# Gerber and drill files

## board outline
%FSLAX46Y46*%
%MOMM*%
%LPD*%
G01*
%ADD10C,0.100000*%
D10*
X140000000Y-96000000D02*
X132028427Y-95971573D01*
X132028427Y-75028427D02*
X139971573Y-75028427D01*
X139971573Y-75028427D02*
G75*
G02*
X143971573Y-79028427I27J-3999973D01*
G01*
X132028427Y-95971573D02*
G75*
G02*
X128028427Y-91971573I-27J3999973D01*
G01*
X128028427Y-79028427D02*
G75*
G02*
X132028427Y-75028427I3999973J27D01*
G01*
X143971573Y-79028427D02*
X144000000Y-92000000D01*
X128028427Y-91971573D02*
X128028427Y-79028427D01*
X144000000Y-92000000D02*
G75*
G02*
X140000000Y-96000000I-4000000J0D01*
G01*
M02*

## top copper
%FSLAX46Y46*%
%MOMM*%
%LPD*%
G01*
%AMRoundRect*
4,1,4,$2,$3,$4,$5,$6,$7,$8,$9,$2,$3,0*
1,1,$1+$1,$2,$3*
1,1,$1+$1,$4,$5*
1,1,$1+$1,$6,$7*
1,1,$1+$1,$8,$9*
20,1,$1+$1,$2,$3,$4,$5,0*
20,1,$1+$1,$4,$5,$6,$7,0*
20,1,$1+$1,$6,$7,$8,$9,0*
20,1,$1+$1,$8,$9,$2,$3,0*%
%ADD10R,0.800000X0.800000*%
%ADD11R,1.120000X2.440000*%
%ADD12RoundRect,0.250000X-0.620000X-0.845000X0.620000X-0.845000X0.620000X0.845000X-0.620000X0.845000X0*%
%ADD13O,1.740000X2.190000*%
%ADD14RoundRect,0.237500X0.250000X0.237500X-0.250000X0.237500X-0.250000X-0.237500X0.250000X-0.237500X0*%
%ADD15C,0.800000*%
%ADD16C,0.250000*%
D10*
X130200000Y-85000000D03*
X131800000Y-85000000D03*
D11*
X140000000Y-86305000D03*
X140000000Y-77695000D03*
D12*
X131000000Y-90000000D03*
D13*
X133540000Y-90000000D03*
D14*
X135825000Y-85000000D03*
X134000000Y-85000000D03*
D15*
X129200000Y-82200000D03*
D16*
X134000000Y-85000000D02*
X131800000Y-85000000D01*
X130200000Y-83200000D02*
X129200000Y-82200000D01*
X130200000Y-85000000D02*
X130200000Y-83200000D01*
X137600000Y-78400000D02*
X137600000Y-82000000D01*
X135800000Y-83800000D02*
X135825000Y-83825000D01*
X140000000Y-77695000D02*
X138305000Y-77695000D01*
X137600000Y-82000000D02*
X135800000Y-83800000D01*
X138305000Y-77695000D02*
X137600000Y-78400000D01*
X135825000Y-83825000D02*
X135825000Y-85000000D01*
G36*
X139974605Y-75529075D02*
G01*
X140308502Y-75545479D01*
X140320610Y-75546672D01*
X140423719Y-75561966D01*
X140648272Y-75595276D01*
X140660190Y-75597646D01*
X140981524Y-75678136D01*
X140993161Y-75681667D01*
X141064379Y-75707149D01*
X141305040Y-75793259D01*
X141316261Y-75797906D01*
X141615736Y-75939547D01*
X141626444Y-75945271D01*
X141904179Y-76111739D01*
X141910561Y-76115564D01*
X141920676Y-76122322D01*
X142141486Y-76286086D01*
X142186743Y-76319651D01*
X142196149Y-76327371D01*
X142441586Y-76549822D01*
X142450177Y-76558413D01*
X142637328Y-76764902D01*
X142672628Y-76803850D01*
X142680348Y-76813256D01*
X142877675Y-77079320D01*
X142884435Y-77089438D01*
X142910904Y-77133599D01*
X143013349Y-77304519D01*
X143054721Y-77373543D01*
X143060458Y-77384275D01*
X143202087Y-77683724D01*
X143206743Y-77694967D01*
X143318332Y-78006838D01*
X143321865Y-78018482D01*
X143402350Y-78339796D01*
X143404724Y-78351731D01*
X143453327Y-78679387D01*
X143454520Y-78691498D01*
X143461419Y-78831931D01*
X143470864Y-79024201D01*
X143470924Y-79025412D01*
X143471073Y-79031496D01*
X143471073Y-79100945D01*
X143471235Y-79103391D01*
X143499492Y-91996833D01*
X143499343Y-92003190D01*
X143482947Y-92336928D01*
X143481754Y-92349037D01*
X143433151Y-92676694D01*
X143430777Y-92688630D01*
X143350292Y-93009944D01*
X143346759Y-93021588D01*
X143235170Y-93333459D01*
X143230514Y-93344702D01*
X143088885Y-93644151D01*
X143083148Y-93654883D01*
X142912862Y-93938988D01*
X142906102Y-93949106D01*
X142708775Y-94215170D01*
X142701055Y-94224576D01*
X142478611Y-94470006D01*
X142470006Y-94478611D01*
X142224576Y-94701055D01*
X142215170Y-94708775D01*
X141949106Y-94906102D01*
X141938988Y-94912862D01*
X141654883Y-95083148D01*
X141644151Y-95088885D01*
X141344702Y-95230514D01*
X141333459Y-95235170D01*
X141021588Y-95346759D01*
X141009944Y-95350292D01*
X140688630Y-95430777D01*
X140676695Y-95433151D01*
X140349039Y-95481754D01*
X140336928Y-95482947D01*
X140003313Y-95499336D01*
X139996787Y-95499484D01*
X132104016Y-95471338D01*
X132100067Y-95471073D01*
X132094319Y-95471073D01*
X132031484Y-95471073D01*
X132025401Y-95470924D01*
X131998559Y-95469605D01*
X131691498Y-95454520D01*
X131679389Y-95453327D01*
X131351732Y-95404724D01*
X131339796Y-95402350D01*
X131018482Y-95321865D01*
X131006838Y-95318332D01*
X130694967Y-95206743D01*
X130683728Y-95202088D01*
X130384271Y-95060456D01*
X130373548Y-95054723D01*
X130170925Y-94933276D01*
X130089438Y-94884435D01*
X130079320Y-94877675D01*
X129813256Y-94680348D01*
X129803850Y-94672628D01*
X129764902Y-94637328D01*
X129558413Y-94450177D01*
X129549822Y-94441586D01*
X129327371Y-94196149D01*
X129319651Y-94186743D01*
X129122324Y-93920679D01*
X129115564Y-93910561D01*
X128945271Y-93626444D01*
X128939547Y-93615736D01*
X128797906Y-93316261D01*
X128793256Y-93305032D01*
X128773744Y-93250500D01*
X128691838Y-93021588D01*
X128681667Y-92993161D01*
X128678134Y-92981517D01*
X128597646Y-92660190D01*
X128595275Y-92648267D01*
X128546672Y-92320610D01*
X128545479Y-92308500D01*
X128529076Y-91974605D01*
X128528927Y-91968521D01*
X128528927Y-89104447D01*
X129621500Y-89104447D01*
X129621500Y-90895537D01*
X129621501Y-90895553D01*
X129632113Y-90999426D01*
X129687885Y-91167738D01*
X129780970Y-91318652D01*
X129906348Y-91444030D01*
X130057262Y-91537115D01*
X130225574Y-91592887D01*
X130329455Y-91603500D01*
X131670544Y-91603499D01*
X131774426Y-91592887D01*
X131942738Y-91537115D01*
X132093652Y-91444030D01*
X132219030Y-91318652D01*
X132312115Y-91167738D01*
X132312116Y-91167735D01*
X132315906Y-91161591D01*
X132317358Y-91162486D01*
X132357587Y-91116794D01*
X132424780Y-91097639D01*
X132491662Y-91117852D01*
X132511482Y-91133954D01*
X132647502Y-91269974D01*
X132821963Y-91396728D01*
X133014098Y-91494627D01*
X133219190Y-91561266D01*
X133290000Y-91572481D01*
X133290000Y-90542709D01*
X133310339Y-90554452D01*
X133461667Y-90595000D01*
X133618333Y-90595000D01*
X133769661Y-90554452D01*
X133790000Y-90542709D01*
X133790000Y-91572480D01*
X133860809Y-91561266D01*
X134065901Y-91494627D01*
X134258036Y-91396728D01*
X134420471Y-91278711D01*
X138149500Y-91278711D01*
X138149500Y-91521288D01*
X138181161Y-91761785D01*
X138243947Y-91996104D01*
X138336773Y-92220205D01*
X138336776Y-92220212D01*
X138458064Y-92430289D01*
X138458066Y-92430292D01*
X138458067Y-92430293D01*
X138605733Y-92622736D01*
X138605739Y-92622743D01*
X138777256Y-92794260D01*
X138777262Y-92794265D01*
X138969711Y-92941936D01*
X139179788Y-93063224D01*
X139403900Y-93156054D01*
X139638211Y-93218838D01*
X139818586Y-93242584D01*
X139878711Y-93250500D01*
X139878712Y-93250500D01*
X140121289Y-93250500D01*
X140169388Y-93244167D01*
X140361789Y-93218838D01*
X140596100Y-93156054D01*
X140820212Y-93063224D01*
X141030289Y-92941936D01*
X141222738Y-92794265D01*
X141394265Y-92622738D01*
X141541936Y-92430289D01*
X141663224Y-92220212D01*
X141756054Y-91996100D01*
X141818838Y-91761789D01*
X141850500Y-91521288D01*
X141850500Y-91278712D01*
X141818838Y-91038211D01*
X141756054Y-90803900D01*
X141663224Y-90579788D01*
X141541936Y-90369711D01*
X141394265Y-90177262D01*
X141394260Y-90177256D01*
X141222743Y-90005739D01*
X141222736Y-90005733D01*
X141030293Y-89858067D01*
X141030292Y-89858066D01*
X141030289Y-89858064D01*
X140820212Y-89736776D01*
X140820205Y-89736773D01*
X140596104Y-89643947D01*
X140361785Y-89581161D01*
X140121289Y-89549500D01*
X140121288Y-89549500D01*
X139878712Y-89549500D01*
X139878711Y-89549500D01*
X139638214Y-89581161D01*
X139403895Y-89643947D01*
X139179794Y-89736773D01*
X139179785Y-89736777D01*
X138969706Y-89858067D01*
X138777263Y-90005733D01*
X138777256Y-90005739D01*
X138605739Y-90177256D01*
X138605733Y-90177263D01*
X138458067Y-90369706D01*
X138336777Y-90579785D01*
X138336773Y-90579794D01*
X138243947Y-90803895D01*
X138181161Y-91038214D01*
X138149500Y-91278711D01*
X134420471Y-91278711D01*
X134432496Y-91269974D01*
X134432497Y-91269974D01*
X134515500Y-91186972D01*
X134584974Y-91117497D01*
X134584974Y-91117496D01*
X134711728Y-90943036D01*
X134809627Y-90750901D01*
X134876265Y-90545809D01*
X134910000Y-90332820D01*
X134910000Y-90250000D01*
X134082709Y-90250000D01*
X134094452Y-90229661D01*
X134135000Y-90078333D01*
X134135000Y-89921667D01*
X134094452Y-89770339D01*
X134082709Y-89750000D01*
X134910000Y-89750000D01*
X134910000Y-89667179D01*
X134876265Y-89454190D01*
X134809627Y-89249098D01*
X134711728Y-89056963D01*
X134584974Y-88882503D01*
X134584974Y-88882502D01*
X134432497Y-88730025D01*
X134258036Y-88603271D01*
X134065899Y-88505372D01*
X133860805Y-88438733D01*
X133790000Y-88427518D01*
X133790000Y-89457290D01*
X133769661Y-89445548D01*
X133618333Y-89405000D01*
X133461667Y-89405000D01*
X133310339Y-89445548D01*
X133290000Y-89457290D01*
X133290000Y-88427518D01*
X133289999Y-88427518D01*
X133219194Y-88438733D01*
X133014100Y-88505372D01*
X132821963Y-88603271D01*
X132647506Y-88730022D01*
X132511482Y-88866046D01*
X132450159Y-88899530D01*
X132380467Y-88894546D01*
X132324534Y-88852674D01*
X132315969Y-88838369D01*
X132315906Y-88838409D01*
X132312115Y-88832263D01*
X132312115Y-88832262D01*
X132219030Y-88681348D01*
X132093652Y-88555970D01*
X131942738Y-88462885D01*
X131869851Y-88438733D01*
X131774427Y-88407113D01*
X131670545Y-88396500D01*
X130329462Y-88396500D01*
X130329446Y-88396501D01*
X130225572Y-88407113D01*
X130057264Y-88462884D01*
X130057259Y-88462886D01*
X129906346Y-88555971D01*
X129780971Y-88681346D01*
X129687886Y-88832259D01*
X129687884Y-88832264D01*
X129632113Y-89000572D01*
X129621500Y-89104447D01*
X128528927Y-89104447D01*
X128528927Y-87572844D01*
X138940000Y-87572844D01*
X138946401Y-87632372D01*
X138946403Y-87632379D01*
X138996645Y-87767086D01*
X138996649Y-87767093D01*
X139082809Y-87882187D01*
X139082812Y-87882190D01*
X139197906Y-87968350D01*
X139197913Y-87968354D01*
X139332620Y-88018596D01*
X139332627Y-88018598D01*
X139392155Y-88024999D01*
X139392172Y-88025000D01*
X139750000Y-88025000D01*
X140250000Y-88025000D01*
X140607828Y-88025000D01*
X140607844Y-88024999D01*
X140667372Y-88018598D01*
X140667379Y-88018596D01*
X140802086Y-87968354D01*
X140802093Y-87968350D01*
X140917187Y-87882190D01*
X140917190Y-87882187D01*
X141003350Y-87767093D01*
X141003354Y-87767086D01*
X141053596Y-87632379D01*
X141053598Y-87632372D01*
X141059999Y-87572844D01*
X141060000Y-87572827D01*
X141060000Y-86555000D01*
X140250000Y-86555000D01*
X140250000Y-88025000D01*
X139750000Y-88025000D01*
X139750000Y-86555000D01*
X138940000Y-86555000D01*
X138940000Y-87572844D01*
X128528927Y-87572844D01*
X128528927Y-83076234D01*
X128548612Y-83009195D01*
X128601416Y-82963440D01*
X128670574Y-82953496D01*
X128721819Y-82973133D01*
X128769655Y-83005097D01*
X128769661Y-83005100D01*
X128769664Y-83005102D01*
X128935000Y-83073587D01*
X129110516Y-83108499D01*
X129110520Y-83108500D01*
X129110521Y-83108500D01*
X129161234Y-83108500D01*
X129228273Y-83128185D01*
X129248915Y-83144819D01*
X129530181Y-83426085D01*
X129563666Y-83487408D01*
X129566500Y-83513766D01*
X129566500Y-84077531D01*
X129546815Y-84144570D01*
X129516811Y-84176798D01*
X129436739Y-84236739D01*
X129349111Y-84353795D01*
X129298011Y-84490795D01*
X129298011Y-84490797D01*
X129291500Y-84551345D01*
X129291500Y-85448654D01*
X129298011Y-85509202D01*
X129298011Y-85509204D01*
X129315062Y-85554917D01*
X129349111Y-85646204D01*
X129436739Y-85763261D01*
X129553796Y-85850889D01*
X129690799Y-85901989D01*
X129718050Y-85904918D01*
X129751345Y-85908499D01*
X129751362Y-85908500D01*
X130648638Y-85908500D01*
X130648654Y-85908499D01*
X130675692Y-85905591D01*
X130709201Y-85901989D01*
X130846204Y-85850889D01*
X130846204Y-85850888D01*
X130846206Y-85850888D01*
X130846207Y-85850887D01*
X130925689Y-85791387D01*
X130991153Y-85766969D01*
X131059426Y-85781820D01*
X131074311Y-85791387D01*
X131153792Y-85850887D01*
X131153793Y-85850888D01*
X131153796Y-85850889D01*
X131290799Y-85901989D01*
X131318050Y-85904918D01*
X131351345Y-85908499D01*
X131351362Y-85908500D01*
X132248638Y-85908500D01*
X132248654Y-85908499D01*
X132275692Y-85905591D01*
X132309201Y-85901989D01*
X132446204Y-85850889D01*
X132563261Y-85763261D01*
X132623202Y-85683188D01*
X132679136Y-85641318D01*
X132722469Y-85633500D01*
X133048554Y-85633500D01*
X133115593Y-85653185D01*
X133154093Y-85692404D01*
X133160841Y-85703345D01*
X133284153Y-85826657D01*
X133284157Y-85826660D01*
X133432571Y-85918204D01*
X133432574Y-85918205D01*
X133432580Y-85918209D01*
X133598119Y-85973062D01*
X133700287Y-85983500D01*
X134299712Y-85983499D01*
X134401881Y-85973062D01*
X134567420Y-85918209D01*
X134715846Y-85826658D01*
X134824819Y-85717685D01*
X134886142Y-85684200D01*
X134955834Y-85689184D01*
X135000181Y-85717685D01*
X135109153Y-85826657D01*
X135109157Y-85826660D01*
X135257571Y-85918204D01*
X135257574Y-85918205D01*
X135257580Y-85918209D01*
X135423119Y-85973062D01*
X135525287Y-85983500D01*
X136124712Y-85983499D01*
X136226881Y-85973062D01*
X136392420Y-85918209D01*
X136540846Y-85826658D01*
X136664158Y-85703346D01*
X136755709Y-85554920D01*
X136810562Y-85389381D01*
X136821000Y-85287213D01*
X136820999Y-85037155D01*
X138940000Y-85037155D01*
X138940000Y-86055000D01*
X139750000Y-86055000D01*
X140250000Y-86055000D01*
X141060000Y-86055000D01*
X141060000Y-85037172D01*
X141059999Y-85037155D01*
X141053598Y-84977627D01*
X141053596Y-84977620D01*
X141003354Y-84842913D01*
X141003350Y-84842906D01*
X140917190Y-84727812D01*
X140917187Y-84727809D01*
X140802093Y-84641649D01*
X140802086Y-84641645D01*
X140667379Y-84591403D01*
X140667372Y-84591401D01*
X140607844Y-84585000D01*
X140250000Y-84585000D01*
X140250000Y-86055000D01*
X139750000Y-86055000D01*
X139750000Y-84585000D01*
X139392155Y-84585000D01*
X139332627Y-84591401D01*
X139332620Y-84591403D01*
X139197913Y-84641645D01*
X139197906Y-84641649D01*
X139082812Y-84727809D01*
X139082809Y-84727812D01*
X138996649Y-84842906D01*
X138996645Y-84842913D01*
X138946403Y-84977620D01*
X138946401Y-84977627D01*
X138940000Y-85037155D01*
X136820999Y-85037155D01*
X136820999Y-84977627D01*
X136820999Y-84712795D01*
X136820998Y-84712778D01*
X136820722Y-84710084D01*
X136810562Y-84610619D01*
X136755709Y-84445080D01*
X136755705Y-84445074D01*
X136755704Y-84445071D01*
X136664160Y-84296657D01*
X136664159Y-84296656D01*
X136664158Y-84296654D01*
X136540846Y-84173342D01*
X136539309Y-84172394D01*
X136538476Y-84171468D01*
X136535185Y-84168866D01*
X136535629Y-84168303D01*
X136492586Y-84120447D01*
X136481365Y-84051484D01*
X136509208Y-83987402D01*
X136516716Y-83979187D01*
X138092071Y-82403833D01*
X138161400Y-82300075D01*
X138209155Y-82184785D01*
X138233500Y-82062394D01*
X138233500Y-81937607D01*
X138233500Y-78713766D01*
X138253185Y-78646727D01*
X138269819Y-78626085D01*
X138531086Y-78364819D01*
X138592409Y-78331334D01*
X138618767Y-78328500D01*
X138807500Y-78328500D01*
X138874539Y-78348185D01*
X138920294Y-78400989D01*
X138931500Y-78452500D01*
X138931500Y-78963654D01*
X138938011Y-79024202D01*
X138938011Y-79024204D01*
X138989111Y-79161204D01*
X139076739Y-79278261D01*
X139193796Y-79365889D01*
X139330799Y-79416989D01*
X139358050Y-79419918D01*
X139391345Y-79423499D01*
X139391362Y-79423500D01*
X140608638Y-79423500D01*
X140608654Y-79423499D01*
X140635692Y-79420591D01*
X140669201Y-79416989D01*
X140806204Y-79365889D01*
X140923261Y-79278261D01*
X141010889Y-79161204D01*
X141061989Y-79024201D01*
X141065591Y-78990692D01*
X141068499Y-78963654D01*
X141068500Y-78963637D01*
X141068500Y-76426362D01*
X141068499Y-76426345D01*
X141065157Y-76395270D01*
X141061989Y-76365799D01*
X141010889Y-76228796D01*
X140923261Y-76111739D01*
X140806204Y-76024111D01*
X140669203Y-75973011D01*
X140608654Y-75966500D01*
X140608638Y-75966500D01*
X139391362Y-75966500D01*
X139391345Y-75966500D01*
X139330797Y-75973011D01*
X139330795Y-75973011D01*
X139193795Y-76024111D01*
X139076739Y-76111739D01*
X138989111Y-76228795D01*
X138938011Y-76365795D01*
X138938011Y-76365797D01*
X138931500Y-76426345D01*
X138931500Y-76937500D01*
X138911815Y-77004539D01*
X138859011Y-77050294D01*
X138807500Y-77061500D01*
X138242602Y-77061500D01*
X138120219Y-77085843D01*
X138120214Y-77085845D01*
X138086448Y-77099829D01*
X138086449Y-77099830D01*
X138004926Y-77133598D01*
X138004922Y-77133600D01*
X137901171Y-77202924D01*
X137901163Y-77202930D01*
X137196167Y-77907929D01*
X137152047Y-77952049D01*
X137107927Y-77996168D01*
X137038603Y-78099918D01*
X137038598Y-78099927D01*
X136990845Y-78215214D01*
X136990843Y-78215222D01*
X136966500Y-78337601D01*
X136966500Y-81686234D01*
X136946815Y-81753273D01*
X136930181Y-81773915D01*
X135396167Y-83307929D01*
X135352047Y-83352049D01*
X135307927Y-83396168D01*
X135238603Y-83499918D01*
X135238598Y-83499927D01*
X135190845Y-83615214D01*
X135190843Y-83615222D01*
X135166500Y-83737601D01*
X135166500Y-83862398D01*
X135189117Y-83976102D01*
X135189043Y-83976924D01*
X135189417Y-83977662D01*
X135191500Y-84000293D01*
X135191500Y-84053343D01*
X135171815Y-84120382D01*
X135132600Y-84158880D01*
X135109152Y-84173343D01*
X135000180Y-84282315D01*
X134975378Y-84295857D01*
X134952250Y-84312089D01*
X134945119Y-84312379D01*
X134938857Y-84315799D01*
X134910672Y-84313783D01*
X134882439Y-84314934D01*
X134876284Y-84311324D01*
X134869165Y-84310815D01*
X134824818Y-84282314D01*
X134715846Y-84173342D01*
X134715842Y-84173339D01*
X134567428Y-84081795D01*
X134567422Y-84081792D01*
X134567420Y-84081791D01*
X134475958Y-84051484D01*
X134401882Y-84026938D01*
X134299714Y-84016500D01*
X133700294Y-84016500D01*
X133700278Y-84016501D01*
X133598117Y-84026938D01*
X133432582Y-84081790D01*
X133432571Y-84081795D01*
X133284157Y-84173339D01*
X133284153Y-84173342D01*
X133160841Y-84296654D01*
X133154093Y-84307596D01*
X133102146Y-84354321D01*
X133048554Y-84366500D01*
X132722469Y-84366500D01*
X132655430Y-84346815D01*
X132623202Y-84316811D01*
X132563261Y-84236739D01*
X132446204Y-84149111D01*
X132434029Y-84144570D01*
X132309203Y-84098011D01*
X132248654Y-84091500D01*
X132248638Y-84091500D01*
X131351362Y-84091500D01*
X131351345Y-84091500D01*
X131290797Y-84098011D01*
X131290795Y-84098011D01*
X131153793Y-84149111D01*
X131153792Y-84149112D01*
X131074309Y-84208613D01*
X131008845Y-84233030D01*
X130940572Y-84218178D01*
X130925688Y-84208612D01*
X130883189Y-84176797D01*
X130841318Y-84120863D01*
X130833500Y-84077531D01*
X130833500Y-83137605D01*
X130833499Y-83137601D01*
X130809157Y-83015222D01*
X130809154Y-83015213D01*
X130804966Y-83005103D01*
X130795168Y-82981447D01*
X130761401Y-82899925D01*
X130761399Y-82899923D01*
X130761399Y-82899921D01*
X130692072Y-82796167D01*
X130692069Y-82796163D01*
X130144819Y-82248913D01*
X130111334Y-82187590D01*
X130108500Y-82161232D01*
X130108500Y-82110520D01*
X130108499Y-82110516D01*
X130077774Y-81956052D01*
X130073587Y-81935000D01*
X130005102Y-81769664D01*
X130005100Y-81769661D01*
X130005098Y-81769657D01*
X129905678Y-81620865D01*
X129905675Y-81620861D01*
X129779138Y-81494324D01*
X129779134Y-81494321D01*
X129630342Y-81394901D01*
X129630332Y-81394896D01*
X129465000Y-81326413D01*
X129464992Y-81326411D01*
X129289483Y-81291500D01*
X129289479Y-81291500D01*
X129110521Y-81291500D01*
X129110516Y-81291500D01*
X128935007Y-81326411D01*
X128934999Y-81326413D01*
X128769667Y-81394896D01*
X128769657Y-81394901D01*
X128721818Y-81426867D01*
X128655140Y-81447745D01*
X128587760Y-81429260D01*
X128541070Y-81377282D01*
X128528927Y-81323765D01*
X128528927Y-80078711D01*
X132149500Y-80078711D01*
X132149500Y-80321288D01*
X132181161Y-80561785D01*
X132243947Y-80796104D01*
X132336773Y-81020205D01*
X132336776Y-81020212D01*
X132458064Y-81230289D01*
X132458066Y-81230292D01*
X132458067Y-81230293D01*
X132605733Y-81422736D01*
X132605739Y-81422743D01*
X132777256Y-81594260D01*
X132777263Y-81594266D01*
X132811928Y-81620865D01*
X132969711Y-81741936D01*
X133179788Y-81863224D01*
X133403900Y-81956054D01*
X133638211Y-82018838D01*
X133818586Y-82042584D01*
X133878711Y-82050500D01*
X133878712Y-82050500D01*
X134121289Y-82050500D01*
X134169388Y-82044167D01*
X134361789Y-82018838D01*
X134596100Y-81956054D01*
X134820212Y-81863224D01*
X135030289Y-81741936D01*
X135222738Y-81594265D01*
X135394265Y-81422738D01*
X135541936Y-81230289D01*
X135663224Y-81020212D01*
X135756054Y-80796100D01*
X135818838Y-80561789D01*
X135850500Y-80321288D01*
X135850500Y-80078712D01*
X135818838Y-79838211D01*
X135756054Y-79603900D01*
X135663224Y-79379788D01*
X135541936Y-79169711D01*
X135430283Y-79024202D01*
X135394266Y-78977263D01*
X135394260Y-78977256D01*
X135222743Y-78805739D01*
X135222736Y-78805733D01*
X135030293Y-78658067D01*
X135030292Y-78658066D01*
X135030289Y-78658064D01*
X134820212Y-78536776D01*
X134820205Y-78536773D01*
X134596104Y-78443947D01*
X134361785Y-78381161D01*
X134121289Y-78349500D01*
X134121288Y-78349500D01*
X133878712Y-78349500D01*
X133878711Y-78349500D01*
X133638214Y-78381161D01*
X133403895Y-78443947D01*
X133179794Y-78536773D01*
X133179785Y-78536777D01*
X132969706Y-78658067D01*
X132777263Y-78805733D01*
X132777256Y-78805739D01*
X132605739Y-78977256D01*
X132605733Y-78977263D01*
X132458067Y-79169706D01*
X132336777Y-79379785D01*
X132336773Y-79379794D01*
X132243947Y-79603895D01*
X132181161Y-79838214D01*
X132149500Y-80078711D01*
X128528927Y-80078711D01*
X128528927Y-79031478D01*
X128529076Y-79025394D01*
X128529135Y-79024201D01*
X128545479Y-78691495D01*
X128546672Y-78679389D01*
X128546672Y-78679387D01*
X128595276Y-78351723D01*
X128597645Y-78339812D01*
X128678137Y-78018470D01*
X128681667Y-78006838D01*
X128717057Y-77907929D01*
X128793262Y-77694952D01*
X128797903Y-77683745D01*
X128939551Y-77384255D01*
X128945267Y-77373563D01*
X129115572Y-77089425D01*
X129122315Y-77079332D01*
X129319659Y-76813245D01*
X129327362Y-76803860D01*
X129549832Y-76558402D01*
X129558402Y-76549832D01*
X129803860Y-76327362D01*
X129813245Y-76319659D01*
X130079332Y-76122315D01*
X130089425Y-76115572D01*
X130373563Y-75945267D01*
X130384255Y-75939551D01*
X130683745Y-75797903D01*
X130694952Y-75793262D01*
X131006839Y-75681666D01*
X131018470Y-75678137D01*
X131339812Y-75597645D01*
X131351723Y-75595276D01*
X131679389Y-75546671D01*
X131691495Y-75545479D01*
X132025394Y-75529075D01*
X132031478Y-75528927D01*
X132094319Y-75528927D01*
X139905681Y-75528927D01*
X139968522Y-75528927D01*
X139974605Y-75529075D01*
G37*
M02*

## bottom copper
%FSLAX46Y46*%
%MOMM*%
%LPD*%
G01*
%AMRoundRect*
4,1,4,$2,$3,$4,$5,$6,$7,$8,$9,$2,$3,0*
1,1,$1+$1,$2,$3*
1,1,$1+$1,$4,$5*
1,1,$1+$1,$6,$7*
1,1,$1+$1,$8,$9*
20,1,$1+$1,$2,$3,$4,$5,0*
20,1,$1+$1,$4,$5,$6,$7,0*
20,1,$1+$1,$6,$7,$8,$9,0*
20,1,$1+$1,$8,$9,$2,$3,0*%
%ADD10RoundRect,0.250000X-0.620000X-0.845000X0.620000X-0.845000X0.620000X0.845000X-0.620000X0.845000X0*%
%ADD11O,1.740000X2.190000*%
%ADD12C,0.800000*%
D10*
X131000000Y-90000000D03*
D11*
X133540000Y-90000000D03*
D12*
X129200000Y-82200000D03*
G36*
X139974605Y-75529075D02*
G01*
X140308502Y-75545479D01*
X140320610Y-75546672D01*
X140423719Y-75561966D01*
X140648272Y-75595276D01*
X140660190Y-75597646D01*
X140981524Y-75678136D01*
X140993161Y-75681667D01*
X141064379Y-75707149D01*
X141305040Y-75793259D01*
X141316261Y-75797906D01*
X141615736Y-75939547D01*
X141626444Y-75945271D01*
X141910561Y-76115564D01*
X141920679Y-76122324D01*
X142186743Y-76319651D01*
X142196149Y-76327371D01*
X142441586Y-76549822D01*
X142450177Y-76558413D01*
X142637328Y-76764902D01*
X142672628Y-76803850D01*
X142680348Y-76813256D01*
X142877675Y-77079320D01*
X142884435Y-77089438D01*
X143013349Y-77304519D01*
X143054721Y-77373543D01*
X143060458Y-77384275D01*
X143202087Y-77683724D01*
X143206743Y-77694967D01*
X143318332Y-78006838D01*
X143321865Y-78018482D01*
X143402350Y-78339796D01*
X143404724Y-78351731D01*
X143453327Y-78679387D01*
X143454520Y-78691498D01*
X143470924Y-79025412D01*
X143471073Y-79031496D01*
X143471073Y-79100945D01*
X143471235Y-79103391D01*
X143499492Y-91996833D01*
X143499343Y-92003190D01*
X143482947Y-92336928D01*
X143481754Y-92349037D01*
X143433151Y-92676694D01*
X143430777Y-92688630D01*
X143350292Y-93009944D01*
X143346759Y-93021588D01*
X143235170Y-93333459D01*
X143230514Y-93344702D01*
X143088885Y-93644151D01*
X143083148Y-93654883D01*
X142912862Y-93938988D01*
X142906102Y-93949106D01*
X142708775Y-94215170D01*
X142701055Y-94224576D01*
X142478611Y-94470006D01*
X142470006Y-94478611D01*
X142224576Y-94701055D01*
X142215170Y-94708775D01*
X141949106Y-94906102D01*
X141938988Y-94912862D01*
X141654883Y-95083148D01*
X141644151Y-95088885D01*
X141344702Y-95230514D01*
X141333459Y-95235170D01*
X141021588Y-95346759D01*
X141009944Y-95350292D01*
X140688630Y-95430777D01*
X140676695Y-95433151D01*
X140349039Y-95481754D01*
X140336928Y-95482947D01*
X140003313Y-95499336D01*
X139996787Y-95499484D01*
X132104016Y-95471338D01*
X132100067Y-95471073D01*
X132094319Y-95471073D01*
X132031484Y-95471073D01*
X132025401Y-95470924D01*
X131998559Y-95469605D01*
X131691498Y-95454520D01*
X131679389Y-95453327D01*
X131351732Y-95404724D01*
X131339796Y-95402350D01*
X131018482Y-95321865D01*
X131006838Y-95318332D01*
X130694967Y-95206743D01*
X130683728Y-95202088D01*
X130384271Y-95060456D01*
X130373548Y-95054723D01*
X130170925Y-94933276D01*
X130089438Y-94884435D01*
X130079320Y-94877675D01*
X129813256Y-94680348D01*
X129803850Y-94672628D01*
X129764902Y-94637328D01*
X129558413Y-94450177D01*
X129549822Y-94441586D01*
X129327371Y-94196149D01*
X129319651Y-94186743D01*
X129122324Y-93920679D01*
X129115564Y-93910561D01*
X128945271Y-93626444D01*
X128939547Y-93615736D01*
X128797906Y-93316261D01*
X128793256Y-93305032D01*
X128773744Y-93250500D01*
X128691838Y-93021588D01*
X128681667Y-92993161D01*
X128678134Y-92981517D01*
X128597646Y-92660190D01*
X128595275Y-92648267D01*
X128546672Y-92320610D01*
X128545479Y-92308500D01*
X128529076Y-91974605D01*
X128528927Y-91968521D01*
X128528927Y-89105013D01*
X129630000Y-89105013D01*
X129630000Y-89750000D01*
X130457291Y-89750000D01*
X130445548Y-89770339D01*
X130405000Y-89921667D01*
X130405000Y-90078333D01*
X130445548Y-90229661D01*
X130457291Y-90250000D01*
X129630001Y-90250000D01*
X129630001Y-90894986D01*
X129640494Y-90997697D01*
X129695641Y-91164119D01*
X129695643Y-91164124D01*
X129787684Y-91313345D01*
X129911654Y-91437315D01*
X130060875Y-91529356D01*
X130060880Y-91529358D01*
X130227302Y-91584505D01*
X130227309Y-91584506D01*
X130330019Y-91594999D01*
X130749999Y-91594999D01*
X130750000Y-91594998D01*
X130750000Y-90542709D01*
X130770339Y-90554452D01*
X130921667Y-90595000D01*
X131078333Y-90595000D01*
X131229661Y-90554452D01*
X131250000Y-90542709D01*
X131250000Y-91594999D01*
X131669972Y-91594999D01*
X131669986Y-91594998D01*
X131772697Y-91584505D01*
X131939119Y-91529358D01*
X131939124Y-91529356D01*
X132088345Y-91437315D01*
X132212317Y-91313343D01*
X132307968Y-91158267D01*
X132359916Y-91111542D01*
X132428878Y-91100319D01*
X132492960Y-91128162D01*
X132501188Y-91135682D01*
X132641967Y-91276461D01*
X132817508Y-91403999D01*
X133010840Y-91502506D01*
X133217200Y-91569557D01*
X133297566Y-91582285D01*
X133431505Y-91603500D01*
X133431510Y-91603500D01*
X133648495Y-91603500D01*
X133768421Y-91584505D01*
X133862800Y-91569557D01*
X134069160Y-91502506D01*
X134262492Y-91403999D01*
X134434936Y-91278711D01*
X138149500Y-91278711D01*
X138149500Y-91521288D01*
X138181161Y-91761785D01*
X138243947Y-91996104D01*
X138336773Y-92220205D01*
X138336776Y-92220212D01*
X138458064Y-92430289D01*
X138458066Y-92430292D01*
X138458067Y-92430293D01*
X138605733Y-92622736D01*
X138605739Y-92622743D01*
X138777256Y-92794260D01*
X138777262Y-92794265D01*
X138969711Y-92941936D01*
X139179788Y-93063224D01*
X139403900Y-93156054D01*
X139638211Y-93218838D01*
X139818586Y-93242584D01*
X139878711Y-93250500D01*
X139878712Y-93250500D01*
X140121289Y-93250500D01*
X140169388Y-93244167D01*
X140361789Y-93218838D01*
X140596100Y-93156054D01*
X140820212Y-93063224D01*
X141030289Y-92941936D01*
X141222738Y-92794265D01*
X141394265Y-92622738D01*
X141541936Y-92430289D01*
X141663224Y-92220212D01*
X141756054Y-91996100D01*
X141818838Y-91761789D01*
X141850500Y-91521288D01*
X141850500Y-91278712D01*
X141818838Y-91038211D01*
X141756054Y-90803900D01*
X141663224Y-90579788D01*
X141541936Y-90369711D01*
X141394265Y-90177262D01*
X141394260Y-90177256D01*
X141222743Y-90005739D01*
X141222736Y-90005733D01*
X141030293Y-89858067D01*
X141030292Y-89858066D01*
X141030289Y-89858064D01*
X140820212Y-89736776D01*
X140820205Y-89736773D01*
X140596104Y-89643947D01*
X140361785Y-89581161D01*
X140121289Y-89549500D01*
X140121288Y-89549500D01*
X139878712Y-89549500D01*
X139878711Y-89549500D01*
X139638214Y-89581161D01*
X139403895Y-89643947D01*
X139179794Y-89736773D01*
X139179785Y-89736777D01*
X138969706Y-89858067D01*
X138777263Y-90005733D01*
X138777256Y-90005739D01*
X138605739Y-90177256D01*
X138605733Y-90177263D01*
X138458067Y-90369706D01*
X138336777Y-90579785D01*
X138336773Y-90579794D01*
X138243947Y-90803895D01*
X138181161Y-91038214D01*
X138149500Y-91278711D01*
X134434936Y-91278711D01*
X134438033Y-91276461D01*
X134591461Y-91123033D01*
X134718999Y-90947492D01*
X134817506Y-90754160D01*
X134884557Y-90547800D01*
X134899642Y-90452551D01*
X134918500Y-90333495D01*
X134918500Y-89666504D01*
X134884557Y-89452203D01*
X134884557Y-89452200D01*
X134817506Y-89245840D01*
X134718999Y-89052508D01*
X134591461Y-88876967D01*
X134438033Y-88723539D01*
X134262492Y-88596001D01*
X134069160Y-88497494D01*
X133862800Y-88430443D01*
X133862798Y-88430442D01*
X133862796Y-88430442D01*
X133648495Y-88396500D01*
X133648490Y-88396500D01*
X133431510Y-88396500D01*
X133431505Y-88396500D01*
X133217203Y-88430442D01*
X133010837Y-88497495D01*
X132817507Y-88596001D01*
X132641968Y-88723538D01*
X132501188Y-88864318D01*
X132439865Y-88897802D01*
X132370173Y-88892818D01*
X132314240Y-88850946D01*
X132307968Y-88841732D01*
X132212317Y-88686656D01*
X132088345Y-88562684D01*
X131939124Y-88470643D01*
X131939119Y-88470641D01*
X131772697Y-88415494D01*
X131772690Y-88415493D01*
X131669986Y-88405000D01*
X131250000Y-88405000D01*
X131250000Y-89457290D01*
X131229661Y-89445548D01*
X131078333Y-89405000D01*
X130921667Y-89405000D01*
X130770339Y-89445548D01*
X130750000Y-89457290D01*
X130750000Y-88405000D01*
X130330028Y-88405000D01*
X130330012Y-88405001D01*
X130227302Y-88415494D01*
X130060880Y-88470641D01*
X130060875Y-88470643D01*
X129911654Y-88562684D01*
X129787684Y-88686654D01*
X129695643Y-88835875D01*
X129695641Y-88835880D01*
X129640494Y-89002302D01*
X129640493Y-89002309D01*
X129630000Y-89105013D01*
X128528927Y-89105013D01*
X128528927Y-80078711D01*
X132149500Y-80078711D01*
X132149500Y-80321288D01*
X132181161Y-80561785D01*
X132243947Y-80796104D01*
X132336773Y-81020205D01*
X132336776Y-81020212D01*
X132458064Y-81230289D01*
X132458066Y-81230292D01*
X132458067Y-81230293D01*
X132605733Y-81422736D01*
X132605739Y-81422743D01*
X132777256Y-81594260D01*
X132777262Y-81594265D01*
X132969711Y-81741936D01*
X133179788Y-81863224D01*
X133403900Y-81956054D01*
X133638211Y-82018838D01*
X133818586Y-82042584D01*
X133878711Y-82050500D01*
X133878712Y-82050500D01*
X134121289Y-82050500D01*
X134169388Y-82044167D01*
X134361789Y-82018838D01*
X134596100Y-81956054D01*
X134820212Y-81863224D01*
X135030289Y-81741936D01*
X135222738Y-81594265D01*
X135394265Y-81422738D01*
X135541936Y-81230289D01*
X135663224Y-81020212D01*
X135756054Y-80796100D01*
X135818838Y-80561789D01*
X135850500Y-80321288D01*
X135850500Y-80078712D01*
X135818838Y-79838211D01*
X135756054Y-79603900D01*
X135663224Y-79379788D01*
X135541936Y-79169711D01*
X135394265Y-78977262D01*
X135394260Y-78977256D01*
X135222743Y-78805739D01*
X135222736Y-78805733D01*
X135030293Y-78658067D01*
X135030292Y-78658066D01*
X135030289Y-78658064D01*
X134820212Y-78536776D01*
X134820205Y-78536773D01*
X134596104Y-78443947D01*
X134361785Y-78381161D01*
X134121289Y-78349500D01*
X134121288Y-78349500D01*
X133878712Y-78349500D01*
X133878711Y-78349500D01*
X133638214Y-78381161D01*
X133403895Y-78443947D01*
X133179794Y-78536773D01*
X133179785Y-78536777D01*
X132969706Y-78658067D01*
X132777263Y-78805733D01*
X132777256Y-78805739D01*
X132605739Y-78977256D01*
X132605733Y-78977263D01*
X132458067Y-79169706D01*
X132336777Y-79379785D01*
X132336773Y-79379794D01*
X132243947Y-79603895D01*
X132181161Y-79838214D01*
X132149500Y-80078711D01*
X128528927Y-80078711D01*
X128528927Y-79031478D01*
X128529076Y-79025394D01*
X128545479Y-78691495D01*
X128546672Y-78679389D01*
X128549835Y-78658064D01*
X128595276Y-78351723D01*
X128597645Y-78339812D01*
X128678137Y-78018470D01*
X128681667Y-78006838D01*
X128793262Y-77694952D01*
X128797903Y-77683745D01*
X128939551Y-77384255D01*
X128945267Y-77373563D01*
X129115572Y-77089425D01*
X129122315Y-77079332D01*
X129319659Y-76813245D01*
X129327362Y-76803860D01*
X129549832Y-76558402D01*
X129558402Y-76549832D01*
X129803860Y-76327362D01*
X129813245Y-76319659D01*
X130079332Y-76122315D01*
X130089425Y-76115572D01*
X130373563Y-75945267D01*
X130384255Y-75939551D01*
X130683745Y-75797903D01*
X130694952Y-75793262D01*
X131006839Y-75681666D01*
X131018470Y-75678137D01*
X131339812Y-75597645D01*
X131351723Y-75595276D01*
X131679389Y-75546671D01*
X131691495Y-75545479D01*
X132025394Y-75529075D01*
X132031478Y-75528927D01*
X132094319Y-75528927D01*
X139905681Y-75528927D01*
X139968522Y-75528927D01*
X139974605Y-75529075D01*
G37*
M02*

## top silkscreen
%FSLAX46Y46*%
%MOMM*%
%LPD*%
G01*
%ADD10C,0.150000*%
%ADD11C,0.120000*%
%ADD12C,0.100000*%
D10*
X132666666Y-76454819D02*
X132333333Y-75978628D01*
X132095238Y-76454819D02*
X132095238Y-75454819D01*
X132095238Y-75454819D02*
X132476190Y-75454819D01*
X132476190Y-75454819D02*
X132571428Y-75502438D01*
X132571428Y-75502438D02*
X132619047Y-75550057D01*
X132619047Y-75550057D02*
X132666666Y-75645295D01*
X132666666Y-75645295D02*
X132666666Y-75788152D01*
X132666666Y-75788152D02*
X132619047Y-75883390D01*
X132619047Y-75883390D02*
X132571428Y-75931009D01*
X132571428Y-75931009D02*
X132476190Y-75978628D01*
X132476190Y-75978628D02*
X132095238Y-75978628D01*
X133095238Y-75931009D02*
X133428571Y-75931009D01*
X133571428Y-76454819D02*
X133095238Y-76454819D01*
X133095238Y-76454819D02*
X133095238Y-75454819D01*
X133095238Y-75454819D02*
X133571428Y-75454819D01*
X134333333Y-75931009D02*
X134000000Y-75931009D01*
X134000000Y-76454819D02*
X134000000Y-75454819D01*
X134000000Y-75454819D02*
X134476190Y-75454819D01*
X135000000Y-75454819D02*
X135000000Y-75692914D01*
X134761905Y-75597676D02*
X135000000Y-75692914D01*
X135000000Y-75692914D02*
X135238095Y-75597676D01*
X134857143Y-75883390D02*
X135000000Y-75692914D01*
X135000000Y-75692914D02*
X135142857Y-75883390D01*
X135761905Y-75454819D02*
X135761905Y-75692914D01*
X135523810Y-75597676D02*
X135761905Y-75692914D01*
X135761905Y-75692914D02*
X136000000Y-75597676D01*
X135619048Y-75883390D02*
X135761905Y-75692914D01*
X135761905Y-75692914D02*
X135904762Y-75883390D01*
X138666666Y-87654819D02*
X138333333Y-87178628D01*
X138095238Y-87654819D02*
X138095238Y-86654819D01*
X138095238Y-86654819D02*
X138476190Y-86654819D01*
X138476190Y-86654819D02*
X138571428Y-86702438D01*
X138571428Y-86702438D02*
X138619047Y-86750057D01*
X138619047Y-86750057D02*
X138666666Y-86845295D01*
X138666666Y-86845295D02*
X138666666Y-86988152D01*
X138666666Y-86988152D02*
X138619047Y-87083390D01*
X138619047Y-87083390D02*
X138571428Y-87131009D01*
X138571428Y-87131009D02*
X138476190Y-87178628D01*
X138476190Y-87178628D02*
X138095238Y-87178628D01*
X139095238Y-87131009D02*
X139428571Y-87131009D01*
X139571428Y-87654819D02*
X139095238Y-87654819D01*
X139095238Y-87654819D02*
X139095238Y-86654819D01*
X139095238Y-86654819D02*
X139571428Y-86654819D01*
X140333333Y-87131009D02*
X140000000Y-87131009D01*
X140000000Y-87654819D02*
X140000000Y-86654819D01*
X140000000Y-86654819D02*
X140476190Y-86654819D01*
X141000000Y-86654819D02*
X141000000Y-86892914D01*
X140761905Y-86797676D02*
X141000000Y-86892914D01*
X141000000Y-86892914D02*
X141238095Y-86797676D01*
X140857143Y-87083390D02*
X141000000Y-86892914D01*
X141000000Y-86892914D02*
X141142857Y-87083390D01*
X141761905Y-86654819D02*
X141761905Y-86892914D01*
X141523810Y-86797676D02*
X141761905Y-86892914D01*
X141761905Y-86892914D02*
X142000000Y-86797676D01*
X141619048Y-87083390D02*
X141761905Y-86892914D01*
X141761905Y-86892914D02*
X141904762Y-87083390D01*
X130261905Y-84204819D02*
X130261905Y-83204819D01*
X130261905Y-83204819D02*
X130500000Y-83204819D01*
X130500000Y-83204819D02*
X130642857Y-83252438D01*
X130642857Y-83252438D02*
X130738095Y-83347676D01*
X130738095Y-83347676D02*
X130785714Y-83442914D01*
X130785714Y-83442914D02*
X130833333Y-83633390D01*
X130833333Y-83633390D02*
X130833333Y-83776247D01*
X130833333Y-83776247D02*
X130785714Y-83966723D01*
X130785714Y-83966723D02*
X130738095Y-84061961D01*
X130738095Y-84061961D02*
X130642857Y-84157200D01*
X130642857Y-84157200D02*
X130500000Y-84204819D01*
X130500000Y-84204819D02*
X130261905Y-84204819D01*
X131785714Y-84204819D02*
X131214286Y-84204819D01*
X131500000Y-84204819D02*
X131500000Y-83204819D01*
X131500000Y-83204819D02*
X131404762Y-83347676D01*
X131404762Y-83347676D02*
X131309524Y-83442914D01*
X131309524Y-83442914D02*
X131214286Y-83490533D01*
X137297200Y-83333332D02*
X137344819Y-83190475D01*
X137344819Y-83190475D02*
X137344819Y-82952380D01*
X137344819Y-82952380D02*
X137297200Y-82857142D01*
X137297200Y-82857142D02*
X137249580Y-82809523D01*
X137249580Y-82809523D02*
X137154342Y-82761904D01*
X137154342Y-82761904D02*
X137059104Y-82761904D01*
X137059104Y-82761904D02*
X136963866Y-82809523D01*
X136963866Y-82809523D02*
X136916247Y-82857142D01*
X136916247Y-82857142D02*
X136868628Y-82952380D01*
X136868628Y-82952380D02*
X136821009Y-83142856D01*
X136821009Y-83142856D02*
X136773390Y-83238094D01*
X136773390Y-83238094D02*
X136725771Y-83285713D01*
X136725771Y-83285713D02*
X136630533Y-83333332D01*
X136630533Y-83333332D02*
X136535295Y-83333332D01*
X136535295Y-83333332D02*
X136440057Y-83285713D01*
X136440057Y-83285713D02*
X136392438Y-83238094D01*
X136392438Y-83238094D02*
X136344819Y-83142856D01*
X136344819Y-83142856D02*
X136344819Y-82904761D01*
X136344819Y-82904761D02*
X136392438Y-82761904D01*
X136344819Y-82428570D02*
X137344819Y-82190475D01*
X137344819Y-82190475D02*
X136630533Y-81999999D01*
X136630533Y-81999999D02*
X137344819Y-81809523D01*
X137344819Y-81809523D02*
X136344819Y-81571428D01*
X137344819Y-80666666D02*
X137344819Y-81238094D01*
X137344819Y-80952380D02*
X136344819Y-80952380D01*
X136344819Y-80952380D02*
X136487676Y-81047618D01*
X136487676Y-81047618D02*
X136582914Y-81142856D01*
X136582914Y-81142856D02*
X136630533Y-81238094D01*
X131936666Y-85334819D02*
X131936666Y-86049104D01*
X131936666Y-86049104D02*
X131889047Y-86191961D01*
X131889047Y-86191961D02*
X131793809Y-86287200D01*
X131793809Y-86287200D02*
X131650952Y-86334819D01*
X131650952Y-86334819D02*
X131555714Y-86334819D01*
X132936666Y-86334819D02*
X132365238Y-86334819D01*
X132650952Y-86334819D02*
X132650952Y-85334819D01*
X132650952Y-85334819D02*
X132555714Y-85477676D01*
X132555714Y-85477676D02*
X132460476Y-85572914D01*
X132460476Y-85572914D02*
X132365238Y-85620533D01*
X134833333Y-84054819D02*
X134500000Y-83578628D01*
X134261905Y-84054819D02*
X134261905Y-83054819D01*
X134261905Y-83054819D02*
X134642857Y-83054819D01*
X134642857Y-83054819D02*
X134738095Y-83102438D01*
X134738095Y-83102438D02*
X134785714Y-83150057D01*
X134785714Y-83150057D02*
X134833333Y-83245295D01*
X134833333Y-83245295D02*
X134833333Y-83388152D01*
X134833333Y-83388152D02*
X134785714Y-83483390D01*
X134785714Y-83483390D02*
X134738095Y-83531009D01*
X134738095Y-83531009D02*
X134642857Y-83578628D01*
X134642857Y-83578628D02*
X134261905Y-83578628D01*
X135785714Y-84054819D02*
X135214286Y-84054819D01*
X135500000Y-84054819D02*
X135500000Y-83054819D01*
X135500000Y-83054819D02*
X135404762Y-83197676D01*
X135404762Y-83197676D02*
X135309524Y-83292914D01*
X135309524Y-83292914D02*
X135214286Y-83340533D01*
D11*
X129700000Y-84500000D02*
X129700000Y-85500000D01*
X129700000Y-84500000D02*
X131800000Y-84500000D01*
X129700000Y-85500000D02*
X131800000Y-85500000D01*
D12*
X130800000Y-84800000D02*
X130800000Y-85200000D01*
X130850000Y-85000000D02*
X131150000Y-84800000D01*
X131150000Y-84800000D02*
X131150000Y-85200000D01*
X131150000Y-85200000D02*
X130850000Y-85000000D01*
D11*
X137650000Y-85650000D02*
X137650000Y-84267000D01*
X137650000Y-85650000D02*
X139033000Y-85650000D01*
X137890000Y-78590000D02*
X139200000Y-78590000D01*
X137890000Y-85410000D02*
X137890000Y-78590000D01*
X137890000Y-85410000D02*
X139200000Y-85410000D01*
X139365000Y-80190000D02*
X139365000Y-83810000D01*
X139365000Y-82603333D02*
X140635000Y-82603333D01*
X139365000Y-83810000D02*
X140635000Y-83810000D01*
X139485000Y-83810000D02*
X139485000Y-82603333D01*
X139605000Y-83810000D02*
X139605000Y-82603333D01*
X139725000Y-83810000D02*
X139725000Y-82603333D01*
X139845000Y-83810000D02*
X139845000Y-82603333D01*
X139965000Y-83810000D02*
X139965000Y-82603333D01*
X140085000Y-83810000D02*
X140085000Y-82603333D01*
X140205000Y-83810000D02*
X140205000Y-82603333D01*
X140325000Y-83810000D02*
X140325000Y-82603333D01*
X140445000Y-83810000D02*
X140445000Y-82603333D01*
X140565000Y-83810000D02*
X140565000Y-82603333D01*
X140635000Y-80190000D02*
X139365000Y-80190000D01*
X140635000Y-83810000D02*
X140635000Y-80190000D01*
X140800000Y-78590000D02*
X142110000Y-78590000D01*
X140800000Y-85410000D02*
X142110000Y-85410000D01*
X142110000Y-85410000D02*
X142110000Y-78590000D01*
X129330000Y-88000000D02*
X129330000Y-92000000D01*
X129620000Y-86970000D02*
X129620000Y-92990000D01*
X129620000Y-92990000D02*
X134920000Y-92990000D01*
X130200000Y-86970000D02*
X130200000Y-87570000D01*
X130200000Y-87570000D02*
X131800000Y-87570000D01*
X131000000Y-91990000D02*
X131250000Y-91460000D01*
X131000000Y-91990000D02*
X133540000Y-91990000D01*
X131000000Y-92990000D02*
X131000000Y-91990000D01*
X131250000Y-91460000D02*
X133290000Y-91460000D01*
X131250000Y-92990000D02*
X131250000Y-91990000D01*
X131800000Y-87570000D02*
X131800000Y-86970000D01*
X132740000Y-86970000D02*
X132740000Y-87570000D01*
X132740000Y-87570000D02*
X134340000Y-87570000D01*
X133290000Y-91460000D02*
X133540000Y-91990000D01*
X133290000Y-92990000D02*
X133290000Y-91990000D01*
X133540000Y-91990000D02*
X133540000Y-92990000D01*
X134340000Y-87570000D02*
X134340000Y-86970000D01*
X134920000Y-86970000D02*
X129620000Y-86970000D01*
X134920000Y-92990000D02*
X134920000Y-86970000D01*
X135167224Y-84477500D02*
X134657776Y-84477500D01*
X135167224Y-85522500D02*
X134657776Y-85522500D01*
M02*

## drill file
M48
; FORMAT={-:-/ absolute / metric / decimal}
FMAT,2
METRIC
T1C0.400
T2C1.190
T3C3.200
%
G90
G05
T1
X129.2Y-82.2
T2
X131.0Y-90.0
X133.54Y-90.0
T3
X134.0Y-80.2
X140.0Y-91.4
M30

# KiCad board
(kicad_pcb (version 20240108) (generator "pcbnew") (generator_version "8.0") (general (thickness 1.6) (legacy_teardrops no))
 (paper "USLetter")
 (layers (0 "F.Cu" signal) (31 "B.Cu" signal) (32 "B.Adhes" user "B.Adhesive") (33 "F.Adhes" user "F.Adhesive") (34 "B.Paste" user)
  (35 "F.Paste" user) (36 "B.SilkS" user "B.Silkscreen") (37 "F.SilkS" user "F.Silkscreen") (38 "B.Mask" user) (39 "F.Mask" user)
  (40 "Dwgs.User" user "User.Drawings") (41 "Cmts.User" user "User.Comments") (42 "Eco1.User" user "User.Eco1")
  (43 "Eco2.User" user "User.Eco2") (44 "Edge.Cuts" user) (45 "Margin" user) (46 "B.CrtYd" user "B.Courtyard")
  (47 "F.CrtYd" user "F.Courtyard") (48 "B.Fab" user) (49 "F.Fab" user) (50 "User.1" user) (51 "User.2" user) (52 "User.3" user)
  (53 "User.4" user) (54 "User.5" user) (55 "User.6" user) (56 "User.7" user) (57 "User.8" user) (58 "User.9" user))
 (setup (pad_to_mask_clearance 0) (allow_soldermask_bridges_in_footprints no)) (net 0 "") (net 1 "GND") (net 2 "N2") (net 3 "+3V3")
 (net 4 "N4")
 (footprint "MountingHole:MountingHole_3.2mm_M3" (layer "F.Cu") (at 134 80.2)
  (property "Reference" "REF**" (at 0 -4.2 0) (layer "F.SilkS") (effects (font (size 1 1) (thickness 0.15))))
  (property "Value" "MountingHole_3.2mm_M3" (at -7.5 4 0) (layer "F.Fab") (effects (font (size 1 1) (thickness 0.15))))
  (pad "" np_thru_hole circle (at 0 0) (size 3.2 3.2) (drill 3.2) (layers "*.Cu" "*.Mask")))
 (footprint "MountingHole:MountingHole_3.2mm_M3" (layer "F.Cu") (at 140 91.4)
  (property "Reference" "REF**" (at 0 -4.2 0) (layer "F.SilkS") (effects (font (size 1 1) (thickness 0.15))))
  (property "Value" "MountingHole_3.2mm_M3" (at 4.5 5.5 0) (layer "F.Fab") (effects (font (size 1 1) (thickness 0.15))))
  (pad "" np_thru_hole circle (at 0 0) (size 3.2 3.2) (drill 3.2) (layers "*.Cu" "*.Mask")))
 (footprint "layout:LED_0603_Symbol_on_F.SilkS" (layer "F.Cu") (at 131 85)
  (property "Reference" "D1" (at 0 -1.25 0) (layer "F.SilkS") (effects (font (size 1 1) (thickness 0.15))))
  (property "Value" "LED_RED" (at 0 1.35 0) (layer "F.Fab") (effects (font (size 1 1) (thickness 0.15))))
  (fp_line (start -1.3 -0.5) (end -1.3 0.5) (stroke (width 0.12) (type solid)) (layer "F.SilkS"))
  (fp_line (start -1.3 -0.5) (end 0.8 -0.5) (stroke (width 0.12) (type solid)) (layer "F.SilkS"))
  (fp_line (start -1.3 0.5) (end 0.8 0.5) (stroke (width 0.12) (type solid)) (layer "F.SilkS"))
  (fp_line (start -0.2 -0.2) (end -0.2 0.2) (stroke (width 0.1) (type solid)) (layer "F.SilkS"))
  (fp_line (start -0.15 0) (end 0.15 -0.2) (stroke (width 0.1) (type solid)) (layer "F.SilkS"))
  (fp_line (start 0.15 -0.2) (end 0.15 0.2) (stroke (width 0.1) (type solid)) (layer "F.SilkS"))
  (fp_line (start 0.15 0.2) (end -0.15 0) (stroke (width 0.1) (type solid)) (layer "F.SilkS"))
  (pad "1" smd rect (at -0.8 0 180) (size 0.8 0.8) (layers "F.Cu" "F.Paste" "F.Mask") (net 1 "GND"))
  (pad "2" smd rect (at 0.8 0 180) (size 0.8 0.8) (layers "F.Cu" "F.Paste" "F.Mask") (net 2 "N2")))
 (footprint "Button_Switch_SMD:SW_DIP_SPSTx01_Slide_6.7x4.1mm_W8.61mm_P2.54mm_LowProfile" (layer "F.Cu") (at 140 82 90)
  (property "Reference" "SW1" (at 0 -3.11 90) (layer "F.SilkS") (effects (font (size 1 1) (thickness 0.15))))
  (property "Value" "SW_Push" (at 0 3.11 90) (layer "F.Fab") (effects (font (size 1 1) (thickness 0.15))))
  (fp_line (start -3.65 -2.35) (end -2.267 -2.35) (stroke (width 0.12) (type solid)) (layer "F.SilkS"))
  (fp_line (start -3.65 -2.35) (end -3.65 -0.967) (stroke (width 0.12) (type solid)) (layer "F.SilkS"))
  (fp_line (start 3.41 -2.11) (end 3.41 -0.8) (stroke (width 0.12) (type solid)) (layer "F.SilkS"))
  (fp_line (start -3.41 -2.11) (end 3.41 -2.11) (stroke (width 0.12) (type solid)) (layer "F.SilkS"))
  (fp_line (start -3.41 -2.11) (end -3.41 -0.8) (stroke (width 0.12) (type solid)) (layer "F.SilkS"))
  (fp_line (start 1.81 -0.635) (end -1.81 -0.635) (stroke (width 0.12) (type solid)) (layer "F.SilkS"))
  (fp_line (start -0.603333 -0.635) (end -0.603333 0.635) (stroke (width 0.12) (type solid)) (layer "F.SilkS"))
  (fp_line (start -1.81 -0.635) (end -1.81 0.635) (stroke (width 0.12) (type solid)) (layer "F.SilkS"))
  (fp_line (start -1.81 -0.515) (end -0.603333 -0.515) (stroke (width 0.12) (type solid)) (layer "F.SilkS"))
  (fp_line (start -1.81 -0.395) (end -0.603333 -0.395) (stroke (width 0.12) (type solid)) (layer "F.SilkS"))
  (fp_line (start -1.81 -0.275) (end -0.603333 -0.275) (stroke (width 0.12) (type solid)) (layer "F.SilkS"))
  (fp_line (start -1.81 -0.155) (end -0.603333 -0.155) (stroke (width 0.12) (type solid)) (layer "F.SilkS"))
  (fp_line (start -1.81 -0.035) (end -0.603333 -0.035) (stroke (width 0.12) (type solid)) (layer "F.SilkS"))
  (fp_line (start -1.81 0.085) (end -0.603333 0.085) (stroke (width 0.12) (type solid)) (layer "F.SilkS"))
  (fp_line (start -1.81 0.205) (end -0.603333 0.205) (stroke (width 0.12) (type solid)) (layer "F.SilkS"))
  (fp_line (start -1.81 0.325) (end -0.603333 0.325) (stroke (width 0.12) (type solid)) (layer "F.SilkS"))
  (fp_line (start -1.81 0.445) (end -0.603333 0.445) (stroke (width 0.12) (type solid)) (layer "F.SilkS"))
  (fp_line (start -1.81 0.565) (end -0.603333 0.565) (stroke (width 0.12) (type solid)) (layer "F.SilkS"))
  (fp_line (start 1.81 0.635) (end 1.81 -0.635) (stroke (width 0.12) (type solid)) (layer "F.SilkS"))
  (fp_line (start -1.81 0.635) (end 1.81 0.635) (stroke (width 0.12) (type solid)) (layer "F.SilkS"))
  (fp_line (start 3.41 0.8) (end 3.41 2.11) (stroke (width 0.12) (type solid)) (layer "F.SilkS"))
  (fp_line (start -3.41 0.8) (end -3.41 2.11) (stroke (width 0.12) (type solid)) (layer "F.SilkS"))
  (fp_line (start -3.41 2.11) (end 3.41 2.11) (stroke (width 0.12) (type solid)) (layer "F.SilkS"))
  (pad "1" smd rect (at -4.305 0 90) (size 2.44 1.12) (layers "F.Cu" "F.Paste" "F.Mask") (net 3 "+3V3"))
  (pad "2" smd rect (at 4.305 0 90) (size 2.44 1.12) (layers "F.Cu" "F.Paste" "F.Mask") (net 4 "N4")))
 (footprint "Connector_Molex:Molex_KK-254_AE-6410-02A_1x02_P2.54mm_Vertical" (layer "F.Cu") (at 131 90)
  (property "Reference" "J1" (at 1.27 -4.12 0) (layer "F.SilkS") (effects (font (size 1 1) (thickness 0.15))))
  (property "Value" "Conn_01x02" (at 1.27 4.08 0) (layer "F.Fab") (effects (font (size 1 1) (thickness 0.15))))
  (fp_line (start -1.67 -2) (end -1.67 2) (stroke (width 0.12) (type solid)) (layer "F.SilkS"))
  (fp_line (start -1.38 -3.03) (end -1.38 2.99) (stroke (width 0.12) (type solid)) (layer "F.SilkS"))
  (fp_line (start -1.38 2.99) (end 3.92 2.99) (stroke (width 0.12) (type solid)) (layer "F.SilkS"))
  (fp_line (start -0.8 -3.03) (end -0.8 -2.43) (stroke (width 0.12) (type solid)) (layer "F.SilkS"))
  (fp_line (start -0.8 -2.43) (end 0.8 -2.43) (stroke (width 0.12) (type solid)) (layer "F.SilkS"))
  (fp_line (start 0 1.99) (end 0.25 1.46) (stroke (width 0.12) (type solid)) (layer "F.SilkS"))
  (fp_line (start 0 1.99) (end 2.54 1.99) (stroke (width 0.12) (type solid)) (layer "F.SilkS"))
  (fp_line (start 0 2.99) (end 0 1.99) (stroke (width 0.12) (type solid)) (layer "F.SilkS"))
  (fp_line (start 0.25 1.46) (end 2.29 1.46) (stroke (width 0.12) (type solid)) (layer "F.SilkS"))
  (fp_line (start 0.25 2.99) (end 0.25 1.99) (stroke (width 0.12) (type solid)) (layer "F.SilkS"))
  (fp_line (start 0.8 -2.43) (end 0.8 -3.03) (stroke (width 0.12) (type solid)) (layer "F.SilkS"))
  (fp_line (start 1.74 -3.03) (end 1.74 -2.43) (stroke (width 0.12) (type solid)) (layer "F.SilkS"))
  (fp_line (start 1.74 -2.43) (end 3.34 -2.43) (stroke (width 0.12) (type solid)) (layer "F.SilkS"))
  (fp_line (start 2.29 1.46) (end 2.54 1.99) (stroke (width 0.12) (type solid)) (layer "F.SilkS"))
  (fp_line (start 2.29 2.99) (end 2.29 1.99) (stroke (width 0.12) (type solid)) (layer "F.SilkS"))
  (fp_line (start 2.54 1.99) (end 2.54 2.99) (stroke (width 0.12) (type solid)) (layer "F.SilkS"))
  (fp_line (start 3.34 -2.43) (end 3.34 -3.03) (stroke (width 0.12) (type solid)) (layer "F.SilkS"))
  (fp_line (start 3.92 -3.03) (end -1.38 -3.03) (stroke (width 0.12) (type solid)) (layer "F.SilkS"))
  (fp_line (start 3.92 2.99) (end 3.92 -3.03) (stroke (width 0.12) (type solid)) (layer "F.SilkS"))
  (pad "1" thru_hole roundrect (at 0 0) (size 1.74 2.19) (drill 1.19) (layers "*.Cu" "*.Mask") (remove_unused_layers no)
   (roundrect_rratio 0.143678) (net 1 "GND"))
  (pad "2" thru_hole oval (at 2.54 0) (size 1.74 2.19) (drill 1.19) (layers "*.Cu" "*.Mask") (remove_unused_layers no) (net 3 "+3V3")))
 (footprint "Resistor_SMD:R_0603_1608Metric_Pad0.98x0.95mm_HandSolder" (layer "F.Cu") (at 134.9125 85 180)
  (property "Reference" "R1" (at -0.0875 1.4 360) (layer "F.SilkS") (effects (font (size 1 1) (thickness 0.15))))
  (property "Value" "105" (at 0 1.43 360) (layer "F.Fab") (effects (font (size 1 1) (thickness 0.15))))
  (fp_line (start -0.254724 0.5225) (end 0.254724 0.5225) (stroke (width 0.12) (type solid)) (layer "F.SilkS"))
  (fp_line (start -0.254724 -0.5225) (end 0.254724 -0.5225) (stroke (width 0.12) (type solid)) (layer "F.SilkS"))
  (pad "1" smd roundrect (at -0.9125 0 180) (size 0.975 0.95) (layers "F.Cu" "F.Paste" "F.Mask") (roundrect_rratio 0.25) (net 4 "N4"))
  (pad "2" smd roundrect (at 0.9125 0 180) (size 0.975 0.95) (layers "F.Cu" "F.Paste" "F.Mask") (roundrect_rratio 0.25) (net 2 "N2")))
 (gr_line (start 140 96) (end 132.028427 95.971573) (stroke (width 0.1) (type default)) (layer "Edge.Cuts"))
 (gr_line (start 132.028427 75.028427) (end 139.971573 75.028427) (stroke (width 0.1) (type default)) (layer "Edge.Cuts"))
 (gr_arc (start 139.971573 75.028427) (mid 142.8 76.2) (end 143.971573 79.028427) (stroke (width 0.1) (type default)) (layer "Edge.Cuts"))
 (gr_arc (start 132.028427 95.971573) (mid 129.2 94.8) (end 128.028427 91.971573) (stroke (width 0.1) (type default)) (layer "Edge.Cuts"))
 (gr_arc (start 128.028427 79.028427) (mid 129.2 76.2) (end 132.028427 75.028427) (stroke (width 0.1) (type default)) (layer "Edge.Cuts"))
 (gr_line (start 143.971573 79.028427) (end 144 92) (stroke (width 0.1) (type default)) (layer "Edge.Cuts"))
 (gr_line (start 128.028427 91.971573) (end 128.028427 79.028427) (stroke (width 0.1) (type default)) (layer "Edge.Cuts"))
 (gr_arc (start 144 92) (mid 142.828427 94.828427) (end 140 96) (stroke (width 0.1) (type default)) (layer "Edge.Cuts"))
 (segment (start 134 85) (end 131.8 85) (width 0.25) (layer "F.Cu") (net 2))
 (segment (start 130.2 83.2) (end 129.2 82.2) (width 0.25) (layer "F.Cu") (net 1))
 (segment (start 130.2 85) (end 130.2 83.2) (width 0.25) (layer "F.Cu") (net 1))
 (via (at 129.2 82.2) (size 0.8) (drill 0.4) (layers "F.Cu" "B.Cu") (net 1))
 (segment (start 137.6 78.4) (end 137.6 82) (width 0.25) (layer "F.Cu") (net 4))
 (segment (start 135.8 83.8) (end 135.825 83.825) (width 0.25) (layer "F.Cu") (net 4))
 (segment (start 140 77.695) (end 138.305 77.695) (width 0.25) (layer "F.Cu") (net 4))
 (segment (start 137.6 82) (end 135.8 83.8) (width 0.25) (layer "F.Cu") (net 4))
 (segment (start 138.305 77.695) (end 137.6 78.4) (width 0.25) (layer "F.Cu") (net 4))
 (segment (start 135.825 83.825) (end 135.825 85) (width 0.25) (layer "F.Cu") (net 4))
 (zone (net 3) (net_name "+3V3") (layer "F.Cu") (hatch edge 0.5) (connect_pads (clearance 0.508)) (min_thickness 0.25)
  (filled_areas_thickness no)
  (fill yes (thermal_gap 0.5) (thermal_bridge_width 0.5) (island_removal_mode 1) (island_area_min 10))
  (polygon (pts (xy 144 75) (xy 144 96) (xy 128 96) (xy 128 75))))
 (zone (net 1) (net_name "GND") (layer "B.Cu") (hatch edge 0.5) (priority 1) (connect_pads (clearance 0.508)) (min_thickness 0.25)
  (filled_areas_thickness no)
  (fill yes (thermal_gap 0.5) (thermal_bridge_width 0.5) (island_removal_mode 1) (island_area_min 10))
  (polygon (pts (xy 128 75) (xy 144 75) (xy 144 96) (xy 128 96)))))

